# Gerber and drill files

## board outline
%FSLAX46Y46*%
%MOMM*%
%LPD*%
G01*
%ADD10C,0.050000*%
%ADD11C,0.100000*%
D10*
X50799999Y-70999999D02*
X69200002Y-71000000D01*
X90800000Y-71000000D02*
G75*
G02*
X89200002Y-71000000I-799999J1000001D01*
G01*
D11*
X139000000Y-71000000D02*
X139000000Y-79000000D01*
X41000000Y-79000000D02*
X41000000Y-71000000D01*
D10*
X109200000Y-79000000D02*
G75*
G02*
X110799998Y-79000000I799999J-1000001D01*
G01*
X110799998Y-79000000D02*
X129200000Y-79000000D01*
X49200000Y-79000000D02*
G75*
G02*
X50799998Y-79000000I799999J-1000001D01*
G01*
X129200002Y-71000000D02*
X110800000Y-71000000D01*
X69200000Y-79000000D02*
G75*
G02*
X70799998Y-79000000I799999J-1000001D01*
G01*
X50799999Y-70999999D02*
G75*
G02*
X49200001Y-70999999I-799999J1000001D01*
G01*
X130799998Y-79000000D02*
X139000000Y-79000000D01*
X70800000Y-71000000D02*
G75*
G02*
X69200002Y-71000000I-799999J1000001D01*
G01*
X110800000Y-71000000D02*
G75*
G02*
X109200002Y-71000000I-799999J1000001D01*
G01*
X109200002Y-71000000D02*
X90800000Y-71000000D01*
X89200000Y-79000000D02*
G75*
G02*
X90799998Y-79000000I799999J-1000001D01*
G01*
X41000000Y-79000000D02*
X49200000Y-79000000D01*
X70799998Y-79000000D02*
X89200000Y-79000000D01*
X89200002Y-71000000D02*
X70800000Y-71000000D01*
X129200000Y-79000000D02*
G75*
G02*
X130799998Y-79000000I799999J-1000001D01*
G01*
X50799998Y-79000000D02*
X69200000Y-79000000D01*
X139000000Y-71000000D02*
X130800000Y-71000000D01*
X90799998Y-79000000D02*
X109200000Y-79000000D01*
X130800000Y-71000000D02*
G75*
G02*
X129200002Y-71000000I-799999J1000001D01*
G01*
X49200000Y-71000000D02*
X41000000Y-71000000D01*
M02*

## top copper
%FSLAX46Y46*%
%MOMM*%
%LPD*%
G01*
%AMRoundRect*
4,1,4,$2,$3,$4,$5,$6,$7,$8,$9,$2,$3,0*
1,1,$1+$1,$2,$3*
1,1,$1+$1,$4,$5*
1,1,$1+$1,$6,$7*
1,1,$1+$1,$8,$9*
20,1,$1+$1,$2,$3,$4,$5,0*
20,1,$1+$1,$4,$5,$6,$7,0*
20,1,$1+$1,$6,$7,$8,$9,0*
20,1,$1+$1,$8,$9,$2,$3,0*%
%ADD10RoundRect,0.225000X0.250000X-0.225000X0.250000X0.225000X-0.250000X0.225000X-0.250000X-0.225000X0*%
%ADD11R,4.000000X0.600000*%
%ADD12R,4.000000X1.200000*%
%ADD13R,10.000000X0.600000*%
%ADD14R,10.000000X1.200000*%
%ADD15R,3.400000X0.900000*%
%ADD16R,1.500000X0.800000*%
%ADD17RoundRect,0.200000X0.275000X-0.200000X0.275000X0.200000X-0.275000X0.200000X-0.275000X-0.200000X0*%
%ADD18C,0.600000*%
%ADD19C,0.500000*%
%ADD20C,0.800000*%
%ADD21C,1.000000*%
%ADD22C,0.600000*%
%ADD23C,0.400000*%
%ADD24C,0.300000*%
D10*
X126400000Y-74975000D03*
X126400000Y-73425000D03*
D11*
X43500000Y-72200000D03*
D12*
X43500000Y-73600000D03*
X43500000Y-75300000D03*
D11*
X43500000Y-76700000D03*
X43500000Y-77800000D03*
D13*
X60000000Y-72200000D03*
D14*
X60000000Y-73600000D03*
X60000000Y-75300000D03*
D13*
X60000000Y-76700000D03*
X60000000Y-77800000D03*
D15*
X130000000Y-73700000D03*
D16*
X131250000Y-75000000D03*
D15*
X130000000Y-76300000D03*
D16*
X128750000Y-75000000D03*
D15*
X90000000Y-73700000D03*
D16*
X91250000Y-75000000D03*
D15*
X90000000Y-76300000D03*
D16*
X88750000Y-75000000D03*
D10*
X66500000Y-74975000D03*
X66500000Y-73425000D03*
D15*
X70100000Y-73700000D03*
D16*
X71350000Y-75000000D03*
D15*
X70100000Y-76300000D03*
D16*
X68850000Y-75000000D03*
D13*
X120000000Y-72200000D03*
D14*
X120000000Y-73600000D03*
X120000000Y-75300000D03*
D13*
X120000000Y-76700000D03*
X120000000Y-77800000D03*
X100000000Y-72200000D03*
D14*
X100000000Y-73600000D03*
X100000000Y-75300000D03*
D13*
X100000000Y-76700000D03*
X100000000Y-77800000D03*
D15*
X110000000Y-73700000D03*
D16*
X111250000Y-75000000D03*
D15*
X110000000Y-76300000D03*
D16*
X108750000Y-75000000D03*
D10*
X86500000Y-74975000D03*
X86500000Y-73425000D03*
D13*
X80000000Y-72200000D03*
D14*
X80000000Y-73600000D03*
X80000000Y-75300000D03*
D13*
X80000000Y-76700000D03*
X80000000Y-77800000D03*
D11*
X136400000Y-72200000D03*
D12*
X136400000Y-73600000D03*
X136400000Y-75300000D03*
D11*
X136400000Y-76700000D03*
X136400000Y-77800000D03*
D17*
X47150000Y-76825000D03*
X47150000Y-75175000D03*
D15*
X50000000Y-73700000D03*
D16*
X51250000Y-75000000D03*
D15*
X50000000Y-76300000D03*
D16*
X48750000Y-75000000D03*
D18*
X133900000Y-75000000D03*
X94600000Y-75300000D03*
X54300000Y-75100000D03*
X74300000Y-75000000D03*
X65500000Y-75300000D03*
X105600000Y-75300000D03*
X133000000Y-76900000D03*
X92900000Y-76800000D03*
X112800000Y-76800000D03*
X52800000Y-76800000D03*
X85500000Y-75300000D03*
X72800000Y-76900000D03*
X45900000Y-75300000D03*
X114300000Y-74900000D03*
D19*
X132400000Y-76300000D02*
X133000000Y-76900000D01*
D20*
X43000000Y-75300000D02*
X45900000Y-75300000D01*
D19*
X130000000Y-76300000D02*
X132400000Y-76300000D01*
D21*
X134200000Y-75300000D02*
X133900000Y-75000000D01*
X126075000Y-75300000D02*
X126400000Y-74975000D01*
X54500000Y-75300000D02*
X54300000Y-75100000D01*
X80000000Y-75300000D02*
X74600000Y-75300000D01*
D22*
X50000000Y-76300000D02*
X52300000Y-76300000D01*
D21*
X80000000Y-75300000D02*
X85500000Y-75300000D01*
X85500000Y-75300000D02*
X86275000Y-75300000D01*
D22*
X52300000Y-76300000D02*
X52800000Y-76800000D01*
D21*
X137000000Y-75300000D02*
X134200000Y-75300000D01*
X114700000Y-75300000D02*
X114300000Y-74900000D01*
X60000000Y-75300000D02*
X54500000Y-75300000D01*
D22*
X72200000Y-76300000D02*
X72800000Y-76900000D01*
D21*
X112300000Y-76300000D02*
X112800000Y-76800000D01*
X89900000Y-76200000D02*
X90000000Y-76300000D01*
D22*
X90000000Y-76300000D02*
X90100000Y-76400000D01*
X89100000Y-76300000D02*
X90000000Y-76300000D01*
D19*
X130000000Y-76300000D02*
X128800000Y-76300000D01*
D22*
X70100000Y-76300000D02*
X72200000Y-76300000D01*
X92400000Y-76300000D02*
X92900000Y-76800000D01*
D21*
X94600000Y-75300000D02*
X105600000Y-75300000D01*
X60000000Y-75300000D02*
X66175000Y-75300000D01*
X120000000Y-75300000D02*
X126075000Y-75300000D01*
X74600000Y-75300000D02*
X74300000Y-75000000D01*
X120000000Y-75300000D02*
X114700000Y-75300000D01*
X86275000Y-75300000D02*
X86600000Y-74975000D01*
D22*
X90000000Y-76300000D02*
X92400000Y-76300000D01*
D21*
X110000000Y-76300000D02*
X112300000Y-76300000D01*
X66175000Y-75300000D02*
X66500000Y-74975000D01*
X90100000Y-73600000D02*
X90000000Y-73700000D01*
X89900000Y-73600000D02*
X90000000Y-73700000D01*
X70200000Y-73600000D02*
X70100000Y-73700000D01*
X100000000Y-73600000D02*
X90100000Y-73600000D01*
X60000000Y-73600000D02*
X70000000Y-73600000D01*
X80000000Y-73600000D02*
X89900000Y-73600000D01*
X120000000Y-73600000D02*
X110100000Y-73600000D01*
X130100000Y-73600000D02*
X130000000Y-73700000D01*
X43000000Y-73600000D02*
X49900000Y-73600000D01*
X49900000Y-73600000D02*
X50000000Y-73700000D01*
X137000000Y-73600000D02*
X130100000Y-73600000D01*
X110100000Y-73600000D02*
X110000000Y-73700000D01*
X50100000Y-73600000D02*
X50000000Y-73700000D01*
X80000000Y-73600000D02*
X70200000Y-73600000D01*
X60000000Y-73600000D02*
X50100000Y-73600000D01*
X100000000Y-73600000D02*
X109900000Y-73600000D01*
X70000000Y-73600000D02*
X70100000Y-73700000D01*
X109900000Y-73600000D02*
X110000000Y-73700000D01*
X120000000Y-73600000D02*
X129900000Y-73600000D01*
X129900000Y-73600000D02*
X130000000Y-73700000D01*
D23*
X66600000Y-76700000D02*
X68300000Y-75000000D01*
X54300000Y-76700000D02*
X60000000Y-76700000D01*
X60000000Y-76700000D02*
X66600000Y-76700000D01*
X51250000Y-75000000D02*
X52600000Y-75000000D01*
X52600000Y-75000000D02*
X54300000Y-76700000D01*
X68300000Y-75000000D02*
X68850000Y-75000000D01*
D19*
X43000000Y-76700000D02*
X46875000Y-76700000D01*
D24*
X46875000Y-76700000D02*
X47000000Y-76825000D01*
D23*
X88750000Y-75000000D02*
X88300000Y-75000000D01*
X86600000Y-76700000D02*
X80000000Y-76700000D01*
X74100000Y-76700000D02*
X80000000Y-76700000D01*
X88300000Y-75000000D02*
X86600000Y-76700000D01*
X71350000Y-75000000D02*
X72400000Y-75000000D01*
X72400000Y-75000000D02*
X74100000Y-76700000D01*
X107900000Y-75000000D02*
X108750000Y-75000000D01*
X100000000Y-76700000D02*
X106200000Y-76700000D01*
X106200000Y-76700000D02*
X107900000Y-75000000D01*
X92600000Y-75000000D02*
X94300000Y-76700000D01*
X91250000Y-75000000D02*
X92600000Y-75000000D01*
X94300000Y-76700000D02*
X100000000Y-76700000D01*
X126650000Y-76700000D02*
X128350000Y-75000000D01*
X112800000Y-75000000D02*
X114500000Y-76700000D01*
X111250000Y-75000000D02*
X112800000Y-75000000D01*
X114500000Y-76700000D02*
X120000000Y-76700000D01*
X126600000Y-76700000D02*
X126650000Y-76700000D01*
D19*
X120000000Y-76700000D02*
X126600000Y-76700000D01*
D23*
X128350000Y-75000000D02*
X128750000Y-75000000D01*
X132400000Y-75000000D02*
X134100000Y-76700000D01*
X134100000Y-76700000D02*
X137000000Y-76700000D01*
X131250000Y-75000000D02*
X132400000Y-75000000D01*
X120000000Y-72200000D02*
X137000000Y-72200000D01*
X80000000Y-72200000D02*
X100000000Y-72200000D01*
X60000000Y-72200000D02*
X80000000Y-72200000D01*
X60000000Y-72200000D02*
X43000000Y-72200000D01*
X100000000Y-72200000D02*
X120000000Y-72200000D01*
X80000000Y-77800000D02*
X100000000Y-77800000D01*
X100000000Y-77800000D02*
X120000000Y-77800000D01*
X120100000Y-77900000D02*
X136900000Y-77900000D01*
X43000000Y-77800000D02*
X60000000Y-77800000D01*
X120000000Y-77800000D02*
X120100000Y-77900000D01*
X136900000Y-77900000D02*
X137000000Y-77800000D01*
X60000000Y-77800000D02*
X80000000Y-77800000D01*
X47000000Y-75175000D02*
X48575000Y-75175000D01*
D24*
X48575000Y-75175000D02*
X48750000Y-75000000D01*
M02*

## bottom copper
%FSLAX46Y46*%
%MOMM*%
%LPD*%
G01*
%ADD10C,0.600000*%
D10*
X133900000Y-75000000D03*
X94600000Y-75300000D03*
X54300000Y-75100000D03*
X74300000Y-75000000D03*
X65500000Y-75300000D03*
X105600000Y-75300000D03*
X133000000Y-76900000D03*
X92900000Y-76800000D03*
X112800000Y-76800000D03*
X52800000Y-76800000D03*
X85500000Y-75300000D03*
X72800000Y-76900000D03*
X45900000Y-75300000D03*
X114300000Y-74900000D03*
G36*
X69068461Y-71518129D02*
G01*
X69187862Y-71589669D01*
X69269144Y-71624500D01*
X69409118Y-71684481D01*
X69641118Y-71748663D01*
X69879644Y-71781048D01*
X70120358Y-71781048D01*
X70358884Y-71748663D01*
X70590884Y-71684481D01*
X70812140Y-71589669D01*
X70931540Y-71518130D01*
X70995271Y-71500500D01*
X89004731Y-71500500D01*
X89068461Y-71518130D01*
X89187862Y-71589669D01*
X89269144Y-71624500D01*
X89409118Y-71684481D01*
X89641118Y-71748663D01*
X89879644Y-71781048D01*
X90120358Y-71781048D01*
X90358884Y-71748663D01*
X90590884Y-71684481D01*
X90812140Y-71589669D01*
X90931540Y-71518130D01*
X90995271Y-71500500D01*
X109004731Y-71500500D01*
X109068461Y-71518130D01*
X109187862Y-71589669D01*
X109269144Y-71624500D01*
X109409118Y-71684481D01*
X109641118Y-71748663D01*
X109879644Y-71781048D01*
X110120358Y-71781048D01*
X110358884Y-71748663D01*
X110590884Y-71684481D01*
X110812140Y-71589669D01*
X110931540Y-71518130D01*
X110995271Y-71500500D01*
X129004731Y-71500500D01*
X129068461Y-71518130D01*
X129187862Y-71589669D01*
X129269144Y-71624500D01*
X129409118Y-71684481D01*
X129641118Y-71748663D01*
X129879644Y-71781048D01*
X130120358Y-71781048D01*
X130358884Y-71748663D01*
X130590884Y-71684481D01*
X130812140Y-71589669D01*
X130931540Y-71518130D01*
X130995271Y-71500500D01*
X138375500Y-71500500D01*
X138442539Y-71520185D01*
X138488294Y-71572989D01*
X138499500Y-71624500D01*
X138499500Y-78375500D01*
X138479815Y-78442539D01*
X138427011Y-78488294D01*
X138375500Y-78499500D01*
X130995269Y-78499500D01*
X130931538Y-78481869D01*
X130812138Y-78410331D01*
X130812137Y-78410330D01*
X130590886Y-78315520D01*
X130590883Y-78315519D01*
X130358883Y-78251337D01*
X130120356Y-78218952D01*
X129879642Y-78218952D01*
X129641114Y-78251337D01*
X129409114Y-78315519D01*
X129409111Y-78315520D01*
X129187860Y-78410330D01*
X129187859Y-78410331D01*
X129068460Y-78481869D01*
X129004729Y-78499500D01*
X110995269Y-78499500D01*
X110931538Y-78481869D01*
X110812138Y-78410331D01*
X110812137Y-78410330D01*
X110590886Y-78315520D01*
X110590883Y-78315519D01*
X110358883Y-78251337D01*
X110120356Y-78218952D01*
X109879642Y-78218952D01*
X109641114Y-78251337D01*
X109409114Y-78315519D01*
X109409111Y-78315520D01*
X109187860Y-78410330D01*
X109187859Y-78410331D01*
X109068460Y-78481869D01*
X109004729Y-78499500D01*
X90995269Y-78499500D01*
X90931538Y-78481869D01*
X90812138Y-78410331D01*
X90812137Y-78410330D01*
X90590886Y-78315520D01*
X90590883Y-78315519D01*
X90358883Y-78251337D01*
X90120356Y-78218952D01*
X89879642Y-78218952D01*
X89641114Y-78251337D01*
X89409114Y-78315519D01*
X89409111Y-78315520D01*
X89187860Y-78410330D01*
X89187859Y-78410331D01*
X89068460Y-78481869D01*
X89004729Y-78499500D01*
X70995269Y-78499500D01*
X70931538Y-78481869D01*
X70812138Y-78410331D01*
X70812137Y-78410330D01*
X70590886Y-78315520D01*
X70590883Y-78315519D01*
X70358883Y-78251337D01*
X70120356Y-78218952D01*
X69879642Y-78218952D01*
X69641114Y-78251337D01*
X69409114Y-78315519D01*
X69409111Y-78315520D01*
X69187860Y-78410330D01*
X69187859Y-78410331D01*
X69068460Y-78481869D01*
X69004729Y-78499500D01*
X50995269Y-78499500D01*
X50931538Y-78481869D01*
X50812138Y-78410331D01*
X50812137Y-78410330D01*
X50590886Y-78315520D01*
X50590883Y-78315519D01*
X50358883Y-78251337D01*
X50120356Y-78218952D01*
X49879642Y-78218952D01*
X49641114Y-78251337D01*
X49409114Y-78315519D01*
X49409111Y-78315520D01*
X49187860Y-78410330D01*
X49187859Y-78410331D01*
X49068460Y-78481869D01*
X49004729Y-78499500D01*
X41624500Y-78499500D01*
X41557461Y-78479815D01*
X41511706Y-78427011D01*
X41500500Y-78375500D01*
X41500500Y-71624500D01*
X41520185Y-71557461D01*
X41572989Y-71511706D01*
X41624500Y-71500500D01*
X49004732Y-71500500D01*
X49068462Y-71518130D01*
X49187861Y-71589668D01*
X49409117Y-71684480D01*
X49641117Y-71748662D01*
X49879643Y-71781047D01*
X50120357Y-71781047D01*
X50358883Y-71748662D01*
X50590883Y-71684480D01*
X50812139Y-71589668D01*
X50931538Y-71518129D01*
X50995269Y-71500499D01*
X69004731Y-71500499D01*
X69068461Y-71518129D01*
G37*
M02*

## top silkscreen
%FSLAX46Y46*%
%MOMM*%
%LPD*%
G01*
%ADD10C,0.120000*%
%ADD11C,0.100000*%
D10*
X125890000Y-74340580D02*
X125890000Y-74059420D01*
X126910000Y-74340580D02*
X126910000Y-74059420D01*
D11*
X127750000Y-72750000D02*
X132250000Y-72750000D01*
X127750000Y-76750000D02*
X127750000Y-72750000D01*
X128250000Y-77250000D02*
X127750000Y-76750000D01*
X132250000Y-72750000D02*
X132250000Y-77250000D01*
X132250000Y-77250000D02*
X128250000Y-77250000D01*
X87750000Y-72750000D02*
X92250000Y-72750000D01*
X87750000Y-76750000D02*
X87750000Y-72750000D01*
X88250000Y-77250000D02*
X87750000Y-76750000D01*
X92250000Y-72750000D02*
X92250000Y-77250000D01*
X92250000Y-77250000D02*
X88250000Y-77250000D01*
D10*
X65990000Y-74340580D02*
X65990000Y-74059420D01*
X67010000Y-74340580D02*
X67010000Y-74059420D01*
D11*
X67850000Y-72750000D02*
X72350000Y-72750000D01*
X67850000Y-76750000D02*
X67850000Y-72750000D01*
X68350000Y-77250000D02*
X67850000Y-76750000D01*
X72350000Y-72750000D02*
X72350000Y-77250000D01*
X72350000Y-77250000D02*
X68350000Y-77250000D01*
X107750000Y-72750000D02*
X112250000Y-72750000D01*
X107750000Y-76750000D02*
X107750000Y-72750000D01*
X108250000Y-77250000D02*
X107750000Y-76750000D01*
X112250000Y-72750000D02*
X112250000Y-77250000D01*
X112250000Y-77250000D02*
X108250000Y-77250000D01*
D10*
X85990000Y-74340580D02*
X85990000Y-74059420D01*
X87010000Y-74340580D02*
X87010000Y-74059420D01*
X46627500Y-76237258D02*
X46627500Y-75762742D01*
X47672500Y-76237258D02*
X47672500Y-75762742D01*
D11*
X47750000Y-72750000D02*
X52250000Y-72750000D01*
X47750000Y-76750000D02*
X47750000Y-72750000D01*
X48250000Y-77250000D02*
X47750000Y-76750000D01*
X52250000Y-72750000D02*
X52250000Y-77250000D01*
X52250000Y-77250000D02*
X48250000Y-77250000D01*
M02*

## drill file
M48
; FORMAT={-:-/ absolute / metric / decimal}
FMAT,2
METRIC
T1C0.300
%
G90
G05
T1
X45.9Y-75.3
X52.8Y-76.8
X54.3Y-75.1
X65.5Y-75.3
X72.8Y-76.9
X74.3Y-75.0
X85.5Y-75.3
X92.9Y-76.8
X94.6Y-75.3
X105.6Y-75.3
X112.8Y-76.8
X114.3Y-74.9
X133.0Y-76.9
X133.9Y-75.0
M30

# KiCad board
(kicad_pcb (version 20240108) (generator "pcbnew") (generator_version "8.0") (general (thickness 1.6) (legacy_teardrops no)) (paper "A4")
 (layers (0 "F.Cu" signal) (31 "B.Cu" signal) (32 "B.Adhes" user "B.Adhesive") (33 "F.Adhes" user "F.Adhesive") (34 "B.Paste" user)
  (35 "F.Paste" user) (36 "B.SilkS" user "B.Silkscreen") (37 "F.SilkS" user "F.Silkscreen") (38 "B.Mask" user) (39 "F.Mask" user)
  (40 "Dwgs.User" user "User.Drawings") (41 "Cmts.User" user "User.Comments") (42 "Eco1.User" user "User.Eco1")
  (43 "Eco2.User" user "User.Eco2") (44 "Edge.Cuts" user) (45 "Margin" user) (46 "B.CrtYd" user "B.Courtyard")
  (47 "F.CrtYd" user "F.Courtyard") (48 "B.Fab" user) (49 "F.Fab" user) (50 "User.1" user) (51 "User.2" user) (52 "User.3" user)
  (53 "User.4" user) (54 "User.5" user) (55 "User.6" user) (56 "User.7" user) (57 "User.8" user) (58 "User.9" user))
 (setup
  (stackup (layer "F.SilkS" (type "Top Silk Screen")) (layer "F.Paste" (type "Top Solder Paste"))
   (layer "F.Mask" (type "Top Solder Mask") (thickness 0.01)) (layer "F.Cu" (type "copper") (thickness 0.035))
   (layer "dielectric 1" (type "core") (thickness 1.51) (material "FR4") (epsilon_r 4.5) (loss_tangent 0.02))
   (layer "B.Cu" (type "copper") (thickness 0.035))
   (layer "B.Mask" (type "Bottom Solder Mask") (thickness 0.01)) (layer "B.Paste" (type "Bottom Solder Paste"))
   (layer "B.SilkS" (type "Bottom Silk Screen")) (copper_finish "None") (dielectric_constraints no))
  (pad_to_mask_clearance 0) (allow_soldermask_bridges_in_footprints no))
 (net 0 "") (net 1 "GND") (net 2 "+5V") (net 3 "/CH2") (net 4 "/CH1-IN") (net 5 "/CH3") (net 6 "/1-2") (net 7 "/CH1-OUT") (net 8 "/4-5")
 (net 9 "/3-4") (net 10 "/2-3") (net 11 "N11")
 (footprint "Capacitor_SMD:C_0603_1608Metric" (layer "F.Cu") (at 126.4 74.2 90)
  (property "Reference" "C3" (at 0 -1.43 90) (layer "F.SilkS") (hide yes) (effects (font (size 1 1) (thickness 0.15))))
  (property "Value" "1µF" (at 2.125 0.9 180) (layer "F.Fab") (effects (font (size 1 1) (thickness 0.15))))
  (fp_line (start -0.14058 -0.51) (end 0.14058 -0.51) (stroke (width 0.12) (type solid)) (layer "F.SilkS"))
  (fp_line (start -0.14058 0.51) (end 0.14058 0.51) (stroke (width 0.12) (type solid)) (layer "F.SilkS"))
  (pad "1" smd roundrect (at -0.775 0 90) (size 0.9 0.95) (layers "F.Cu" "F.Paste" "F.Mask") (roundrect_rratio 0.25) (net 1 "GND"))
  (pad "2" smd roundrect (at 0.775 0 90) (size 0.9 0.95) (layers "F.Cu" "F.Paste" "F.Mask") (roundrect_rratio 0.25) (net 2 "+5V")))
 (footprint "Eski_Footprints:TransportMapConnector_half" (layer "F.Cu") (at 43.5 75)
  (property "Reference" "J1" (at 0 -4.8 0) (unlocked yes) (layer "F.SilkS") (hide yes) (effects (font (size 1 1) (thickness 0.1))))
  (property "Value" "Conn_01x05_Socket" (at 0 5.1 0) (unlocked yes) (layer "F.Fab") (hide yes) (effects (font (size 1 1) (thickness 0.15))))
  (pad "1" smd rect (at 0 -2.8) (size 4 0.6) (layers "F.Cu" "F.Paste" "F.Mask") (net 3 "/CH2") (thermal_bridge_angle 45))
  (pad "2" smd rect (at 0 -1.4) (size 4 1.2) (layers "F.Cu" "F.Paste" "F.Mask") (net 2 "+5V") (thermal_bridge_angle 45))
  (pad "3" smd rect (at 0 0.3) (size 4 1.2) (layers "F.Cu" "F.Paste" "F.Mask") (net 1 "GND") (thermal_bridge_angle 45))
  (pad "4" smd rect (at 0 1.7) (size 4 0.6) (layers "F.Cu" "F.Paste" "F.Mask") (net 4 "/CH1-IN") (thermal_bridge_angle 45))
  (pad "5" smd rect (at 0 2.8) (size 4 0.6) (layers "F.Cu" "F.Paste" "F.Mask") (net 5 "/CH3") (thermal_bridge_angle 45)))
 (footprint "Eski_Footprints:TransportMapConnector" (layer "F.Cu") (at 60 75)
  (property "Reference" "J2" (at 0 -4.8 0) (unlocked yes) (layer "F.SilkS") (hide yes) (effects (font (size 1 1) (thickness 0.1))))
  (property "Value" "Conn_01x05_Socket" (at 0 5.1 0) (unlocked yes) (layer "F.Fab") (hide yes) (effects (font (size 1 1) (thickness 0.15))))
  (pad "1" smd rect (at 0 -2.8) (size 10 0.6) (layers "F.Cu" "F.Paste" "F.Mask") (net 3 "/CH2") (thermal_bridge_angle 45))
  (pad "2" smd rect (at 0 -1.4) (size 10 1.2) (layers "F.Cu" "F.Paste" "F.Mask") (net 2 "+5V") (thermal_bridge_angle 45))
  (pad "3" smd rect (at 0 0.3) (size 10 1.2) (layers "F.Cu" "F.Paste" "F.Mask") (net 1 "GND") (thermal_bridge_angle 45))
  (pad "4" smd rect (at 0 1.7) (size 10 0.6) (layers "F.Cu" "F.Paste" "F.Mask") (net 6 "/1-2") (thermal_bridge_angle 45))
  (pad "5" smd rect (at 0 2.8) (size 10 0.6) (layers "F.Cu" "F.Paste" "F.Mask") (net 5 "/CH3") (thermal_bridge_angle 45)))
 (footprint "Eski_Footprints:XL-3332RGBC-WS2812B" (layer "F.Cu") (at 130 75)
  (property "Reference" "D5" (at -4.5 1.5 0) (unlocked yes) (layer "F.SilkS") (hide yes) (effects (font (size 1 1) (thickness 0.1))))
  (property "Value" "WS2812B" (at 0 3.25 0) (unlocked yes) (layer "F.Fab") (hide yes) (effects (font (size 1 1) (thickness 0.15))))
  (fp_line (start -2.25 -2.25) (end 2.25 -2.25) (stroke (width 0.1) (type default)) (layer "F.SilkS"))
  (fp_line (start -2.25 1.75) (end -2.25 -2.25) (stroke (width 0.1) (type default)) (layer "F.SilkS"))
  (fp_line (start -1.75 2.25) (end -2.25 1.75) (stroke (width 0.1) (type default)) (layer "F.SilkS"))
  (fp_line (start 2.25 -2.25) (end 2.25 2.25) (stroke (width 0.1) (type default)) (layer "F.SilkS"))
  (fp_line (start 2.25 2.25) (end -1.75 2.25) (stroke (width 0.1) (type default)) (layer "F.SilkS"))
  (pad "1" smd rect (at 0 -1.3) (size 3.4 0.9) (layers "F.Cu" "F.Paste" "F.Mask") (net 2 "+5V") (thermal_bridge_angle 45))
  (pad "2" smd rect (at 1.25 0) (size 1.5 0.8) (layers "F.Cu" "F.Paste" "F.Mask") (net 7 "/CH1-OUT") (thermal_bridge_angle 45))
  (pad "3" smd rect (at 0 1.3) (size 3.4 0.9) (layers "F.Cu" "F.Paste" "F.Mask") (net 1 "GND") (thermal_bridge_angle 45))
  (pad "4" smd rect (at -1.25 0) (size 1.5 0.8) (layers "F.Cu" "F.Paste" "F.Mask") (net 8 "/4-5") (thermal_bridge_angle 45)))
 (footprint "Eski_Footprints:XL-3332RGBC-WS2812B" (layer "F.Cu") (at 90 75)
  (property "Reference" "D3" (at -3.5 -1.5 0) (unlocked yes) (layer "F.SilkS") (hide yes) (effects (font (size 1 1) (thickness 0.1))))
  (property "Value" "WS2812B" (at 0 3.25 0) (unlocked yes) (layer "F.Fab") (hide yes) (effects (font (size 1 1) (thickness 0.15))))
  (fp_line (start -2.25 -2.25) (end 2.25 -2.25) (stroke (width 0.1) (type default)) (layer "F.SilkS"))
  (fp_line (start -2.25 1.75) (end -2.25 -2.25) (stroke (width 0.1) (type default)) (layer "F.SilkS"))
  (fp_line (start -1.75 2.25) (end -2.25 1.75) (stroke (width 0.1) (type default)) (layer "F.SilkS"))
  (fp_line (start 2.25 -2.25) (end 2.25 2.25) (stroke (width 0.1) (type default)) (layer "F.SilkS"))
  (fp_line (start 2.25 2.25) (end -1.75 2.25) (stroke (width 0.1) (type default)) (layer "F.SilkS"))
  (pad "1" smd rect (at 0 -1.3) (size 3.4 0.9) (layers "F.Cu" "F.Paste" "F.Mask") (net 2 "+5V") (thermal_bridge_angle 45))
  (pad "2" smd rect (at 1.25 0) (size 1.5 0.8) (layers "F.Cu" "F.Paste" "F.Mask") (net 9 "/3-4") (thermal_bridge_angle 45))
  (pad "3" smd rect (at 0 1.3) (size 3.4 0.9) (layers "F.Cu" "F.Paste" "F.Mask") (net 1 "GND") (thermal_bridge_angle 45))
  (pad "4" smd rect (at -1.25 0) (size 1.5 0.8) (layers "F.Cu" "F.Paste" "F.Mask") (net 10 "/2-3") (thermal_bridge_angle 45)))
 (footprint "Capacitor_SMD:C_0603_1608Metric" (layer "F.Cu") (at 66.5 74.2 90)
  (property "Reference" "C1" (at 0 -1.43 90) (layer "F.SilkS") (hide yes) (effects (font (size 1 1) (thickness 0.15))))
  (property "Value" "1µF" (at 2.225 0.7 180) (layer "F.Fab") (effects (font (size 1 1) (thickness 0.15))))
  (fp_line (start -0.14058 -0.51) (end 0.14058 -0.51) (stroke (width 0.12) (type solid)) (layer "F.SilkS"))
  (fp_line (start -0.14058 0.51) (end 0.14058 0.51) (stroke (width 0.12) (type solid)) (layer "F.SilkS"))
  (pad "1" smd roundrect (at -0.775 0 90) (size 0.9 0.95) (layers "F.Cu" "F.Paste" "F.Mask") (roundrect_rratio 0.25) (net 1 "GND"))
  (pad "2" smd roundrect (at 0.775 0 90) (size 0.9 0.95) (layers "F.Cu" "F.Paste" "F.Mask") (roundrect_rratio 0.25) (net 2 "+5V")))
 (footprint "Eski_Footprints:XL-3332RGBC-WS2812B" (layer "F.Cu") (at 70.1 75)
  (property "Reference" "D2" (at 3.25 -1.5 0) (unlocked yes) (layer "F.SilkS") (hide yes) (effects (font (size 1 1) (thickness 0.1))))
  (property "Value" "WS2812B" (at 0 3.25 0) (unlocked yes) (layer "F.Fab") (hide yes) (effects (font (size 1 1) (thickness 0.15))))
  (fp_line (start -2.25 -2.25) (end 2.25 -2.25) (stroke (width 0.1) (type default)) (layer "F.SilkS"))
  (fp_line (start -2.25 1.75) (end -2.25 -2.25) (stroke (width 0.1) (type default)) (layer "F.SilkS"))
  (fp_line (start -1.75 2.25) (end -2.25 1.75) (stroke (width 0.1) (type default)) (layer "F.SilkS"))
  (fp_line (start 2.25 -2.25) (end 2.25 2.25) (stroke (width 0.1) (type default)) (layer "F.SilkS"))
  (fp_line (start 2.25 2.25) (end -1.75 2.25) (stroke (width 0.1) (type default)) (layer "F.SilkS"))
  (pad "1" smd rect (at 0 -1.3) (size 3.4 0.9) (layers "F.Cu" "F.Paste" "F.Mask") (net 2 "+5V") (thermal_bridge_angle 45))
  (pad "2" smd rect (at 1.25 0) (size 1.5 0.8) (layers "F.Cu" "F.Paste" "F.Mask") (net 10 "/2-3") (thermal_bridge_angle 45))
  (pad "3" smd rect (at 0 1.3) (size 3.4 0.9) (layers "F.Cu" "F.Paste" "F.Mask") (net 1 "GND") (thermal_bridge_angle 45))
  (pad "4" smd rect (at -1.25 0) (size 1.5 0.8) (layers "F.Cu" "F.Paste" "F.Mask") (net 6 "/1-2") (thermal_bridge_angle 45)))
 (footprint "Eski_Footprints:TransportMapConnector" (layer "F.Cu") (at 120 75)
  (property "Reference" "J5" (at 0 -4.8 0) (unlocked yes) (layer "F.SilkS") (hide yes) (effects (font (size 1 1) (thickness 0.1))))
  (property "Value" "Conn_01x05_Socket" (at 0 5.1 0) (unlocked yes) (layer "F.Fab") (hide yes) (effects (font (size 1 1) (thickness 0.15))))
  (pad "1" smd rect (at 0 -2.8) (size 10 0.6) (layers "F.Cu" "F.Paste" "F.Mask") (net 3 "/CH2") (thermal_bridge_angle 45))
  (pad "2" smd rect (at 0 -1.4) (size 10 1.2) (layers "F.Cu" "F.Paste" "F.Mask") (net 2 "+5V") (thermal_bridge_angle 45))
  (pad "3" smd rect (at 0 0.3) (size 10 1.2) (layers "F.Cu" "F.Paste" "F.Mask") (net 1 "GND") (thermal_bridge_angle 45))
  (pad "4" smd rect (at 0 1.7) (size 10 0.6) (layers "F.Cu" "F.Paste" "F.Mask") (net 8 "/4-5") (thermal_bridge_angle 45))
  (pad "5" smd rect (at 0 2.8) (size 10 0.6) (layers "F.Cu" "F.Paste" "F.Mask") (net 5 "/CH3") (thermal_bridge_angle 45)))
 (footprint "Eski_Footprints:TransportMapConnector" (layer "F.Cu") (at 100 75)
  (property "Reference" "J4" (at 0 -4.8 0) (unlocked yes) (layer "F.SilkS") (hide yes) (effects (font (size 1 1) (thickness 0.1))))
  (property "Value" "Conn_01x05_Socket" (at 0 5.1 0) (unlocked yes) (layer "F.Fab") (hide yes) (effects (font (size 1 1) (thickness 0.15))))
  (pad "1" smd rect (at 0 -2.8) (size 10 0.6) (layers "F.Cu" "F.Paste" "F.Mask") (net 3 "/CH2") (thermal_bridge_angle 45))
  (pad "2" smd rect (at 0 -1.4) (size 10 1.2) (layers "F.Cu" "F.Paste" "F.Mask") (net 2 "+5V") (thermal_bridge_angle 45))
  (pad "3" smd rect (at 0 0.3) (size 10 1.2) (layers "F.Cu" "F.Paste" "F.Mask") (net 1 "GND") (thermal_bridge_angle 45))
  (pad "4" smd rect (at 0 1.7) (size 10 0.6) (layers "F.Cu" "F.Paste" "F.Mask") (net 9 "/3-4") (thermal_bridge_angle 45))
  (pad "5" smd rect (at 0 2.8) (size 10 0.6) (layers "F.Cu" "F.Paste" "F.Mask") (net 5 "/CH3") (thermal_bridge_angle 45)))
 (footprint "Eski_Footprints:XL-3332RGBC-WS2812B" (layer "F.Cu") (at 110 75)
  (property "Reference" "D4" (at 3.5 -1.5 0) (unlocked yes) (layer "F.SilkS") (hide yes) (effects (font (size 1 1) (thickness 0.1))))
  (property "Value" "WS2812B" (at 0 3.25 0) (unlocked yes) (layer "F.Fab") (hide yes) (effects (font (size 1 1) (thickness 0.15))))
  (fp_line (start -2.25 -2.25) (end 2.25 -2.25) (stroke (width 0.1) (type default)) (layer "F.SilkS"))
  (fp_line (start -2.25 1.75) (end -2.25 -2.25) (stroke (width 0.1) (type default)) (layer "F.SilkS"))
  (fp_line (start -1.75 2.25) (end -2.25 1.75) (stroke (width 0.1) (type default)) (layer "F.SilkS"))
  (fp_line (start 2.25 -2.25) (end 2.25 2.25) (stroke (width 0.1) (type default)) (layer "F.SilkS"))
  (fp_line (start 2.25 2.25) (end -1.75 2.25) (stroke (width 0.1) (type default)) (layer "F.SilkS"))
  (pad "1" smd rect (at 0 -1.3) (size 3.4 0.9) (layers "F.Cu" "F.Paste" "F.Mask") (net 2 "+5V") (thermal_bridge_angle 45))
  (pad "2" smd rect (at 1.25 0) (size 1.5 0.8) (layers "F.Cu" "F.Paste" "F.Mask") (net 8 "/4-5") (thermal_bridge_angle 45))
  (pad "3" smd rect (at 0 1.3) (size 3.4 0.9) (layers "F.Cu" "F.Paste" "F.Mask") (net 1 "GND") (thermal_bridge_angle 45))
  (pad "4" smd rect (at -1.25 0) (size 1.5 0.8) (layers "F.Cu" "F.Paste" "F.Mask") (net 9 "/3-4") (thermal_bridge_angle 45)))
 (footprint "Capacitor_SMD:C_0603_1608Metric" (layer "F.Cu") (at 86.5 74.2 90)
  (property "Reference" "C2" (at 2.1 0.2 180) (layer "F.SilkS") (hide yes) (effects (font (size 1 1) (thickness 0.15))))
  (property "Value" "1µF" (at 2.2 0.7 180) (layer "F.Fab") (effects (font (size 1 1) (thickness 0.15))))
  (fp_line (start -0.14058 -0.51) (end 0.14058 -0.51) (stroke (width 0.12) (type solid)) (layer "F.SilkS"))
  (fp_line (start -0.14058 0.51) (end 0.14058 0.51) (stroke (width 0.12) (type solid)) (layer "F.SilkS"))
  (pad "1" smd roundrect (at -0.775 0 90) (size 0.9 0.95) (layers "F.Cu" "F.Paste" "F.Mask") (roundrect_rratio 0.25) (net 1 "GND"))
  (pad "2" smd roundrect (at 0.775 0 90) (size 0.9 0.95) (layers "F.Cu" "F.Paste" "F.Mask") (roundrect_rratio 0.25) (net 2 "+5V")))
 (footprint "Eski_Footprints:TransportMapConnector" (layer "F.Cu") (at 80 75)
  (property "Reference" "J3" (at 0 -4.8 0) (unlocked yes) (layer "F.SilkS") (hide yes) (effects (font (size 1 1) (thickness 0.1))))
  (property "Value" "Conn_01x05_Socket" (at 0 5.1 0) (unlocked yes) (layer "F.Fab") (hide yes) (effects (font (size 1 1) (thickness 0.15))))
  (pad "1" smd rect (at 0 -2.8) (size 10 0.6) (layers "F.Cu" "F.Paste" "F.Mask") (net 3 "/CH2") (thermal_bridge_angle 45))
  (pad "2" smd rect (at 0 -1.4) (size 10 1.2) (layers "F.Cu" "F.Paste" "F.Mask") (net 2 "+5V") (thermal_bridge_angle 45))
  (pad "3" smd rect (at 0 0.3) (size 10 1.2) (layers "F.Cu" "F.Paste" "F.Mask") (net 1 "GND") (thermal_bridge_angle 45))
  (pad "4" smd rect (at 0 1.7) (size 10 0.6) (layers "F.Cu" "F.Paste" "F.Mask") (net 10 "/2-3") (thermal_bridge_angle 45))
  (pad "5" smd rect (at 0 2.8) (size 10 0.6) (layers "F.Cu" "F.Paste" "F.Mask") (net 5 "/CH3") (thermal_bridge_angle 45)))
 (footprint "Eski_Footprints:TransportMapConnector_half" (layer "F.Cu") (at 136.4 75)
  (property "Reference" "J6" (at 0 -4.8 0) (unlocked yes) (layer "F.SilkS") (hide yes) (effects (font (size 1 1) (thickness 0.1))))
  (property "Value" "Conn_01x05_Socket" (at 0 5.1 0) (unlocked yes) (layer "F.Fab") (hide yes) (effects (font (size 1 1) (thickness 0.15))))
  (pad "1" smd rect (at 0 -2.8) (size 4 0.6) (layers "F.Cu" "F.Paste" "F.Mask") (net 3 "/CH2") (thermal_bridge_angle 45))
  (pad "2" smd rect (at 0 -1.4) (size 4 1.2) (layers "F.Cu" "F.Paste" "F.Mask") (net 2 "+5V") (thermal_bridge_angle 45))
  (pad "3" smd rect (at 0 0.3) (size 4 1.2) (layers "F.Cu" "F.Paste" "F.Mask") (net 1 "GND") (thermal_bridge_angle 45))
  (pad "4" smd rect (at 0 1.7) (size 4 0.6) (layers "F.Cu" "F.Paste" "F.Mask") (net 7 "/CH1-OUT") (thermal_bridge_angle 45))
  (pad "5" smd rect (at 0 2.8) (size 4 0.6) (layers "F.Cu" "F.Paste" "F.Mask") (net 5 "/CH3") (thermal_bridge_angle 45)))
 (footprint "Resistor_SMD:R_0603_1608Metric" (layer "F.Cu") (at 47.15 76 90)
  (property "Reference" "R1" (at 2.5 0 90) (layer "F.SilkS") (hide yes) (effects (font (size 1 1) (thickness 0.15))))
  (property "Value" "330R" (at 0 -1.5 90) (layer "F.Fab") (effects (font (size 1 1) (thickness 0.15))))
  (fp_line (start -0.237258 -0.5225) (end 0.237258 -0.5225) (stroke (width 0.12) (type solid)) (layer "F.SilkS"))
  (fp_line (start -0.237258 0.5225) (end 0.237258 0.5225) (stroke (width 0.12) (type solid)) (layer "F.SilkS"))
  (pad "1" smd roundrect (at -0.825 0 90) (size 0.8 0.95) (layers "F.Cu" "F.Paste" "F.Mask") (roundrect_rratio 0.25) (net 4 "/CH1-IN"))
  (pad "2" smd roundrect (at 0.825 0 90) (size 0.8 0.95) (layers "F.Cu" "F.Paste" "F.Mask") (roundrect_rratio 0.25) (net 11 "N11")))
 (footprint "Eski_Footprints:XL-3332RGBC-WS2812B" (layer "F.Cu") (at 50 75)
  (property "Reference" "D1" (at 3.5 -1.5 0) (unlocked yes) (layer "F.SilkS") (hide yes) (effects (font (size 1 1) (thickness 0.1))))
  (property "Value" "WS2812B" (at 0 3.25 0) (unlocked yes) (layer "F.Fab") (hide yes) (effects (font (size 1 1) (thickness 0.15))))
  (fp_line (start -2.25 -2.25) (end 2.25 -2.25) (stroke (width 0.1) (type default)) (layer "F.SilkS"))
  (fp_line (start -2.25 1.75) (end -2.25 -2.25) (stroke (width 0.1) (type default)) (layer "F.SilkS"))
  (fp_line (start -1.75 2.25) (end -2.25 1.75) (stroke (width 0.1) (type default)) (layer "F.SilkS"))
  (fp_line (start 2.25 -2.25) (end 2.25 2.25) (stroke (width 0.1) (type default)) (layer "F.SilkS"))
  (fp_line (start 2.25 2.25) (end -1.75 2.25) (stroke (width 0.1) (type default)) (layer "F.SilkS"))
  (pad "1" smd rect (at 0 -1.3) (size 3.4 0.9) (layers "F.Cu" "F.Paste" "F.Mask") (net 2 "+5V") (thermal_bridge_angle 45))
  (pad "2" smd rect (at 1.25 0) (size 1.5 0.8) (layers "F.Cu" "F.Paste" "F.Mask") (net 6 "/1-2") (thermal_bridge_angle 45))
  (pad "3" smd rect (at 0 1.3) (size 3.4 0.9) (layers "F.Cu" "F.Paste" "F.Mask") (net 1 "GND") (thermal_bridge_angle 45))
  (pad "4" smd rect (at -1.25 0) (size 1.5 0.8) (layers "F.Cu" "F.Paste" "F.Mask") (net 11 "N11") (thermal_bridge_angle 45)))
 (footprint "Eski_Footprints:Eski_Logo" (layer "B.Cu") (at 60.1 76.6 180)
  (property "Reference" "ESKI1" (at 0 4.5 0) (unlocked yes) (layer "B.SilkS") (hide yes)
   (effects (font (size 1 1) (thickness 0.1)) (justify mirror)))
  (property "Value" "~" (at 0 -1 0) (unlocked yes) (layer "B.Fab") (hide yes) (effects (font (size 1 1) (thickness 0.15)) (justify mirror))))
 (gr_line (start 50.799999 70.999999) (end 69.200002 71) (stroke (width 0.05) (type default)) (layer "Edge.Cuts"))
 (gr_arc (start 90.8 71) (mid 90.000001 71.280624) (end 89.200002 71) (stroke (width 0.05) (type default)) (layer "Edge.Cuts"))
 (gr_line (start 139 71) (end 139 79) (stroke (width 0.1) (type default)) (layer "Edge.Cuts"))
 (gr_line (start 41 79) (end 41 71) (stroke (width 0.1) (type default)) (layer "Edge.Cuts"))
 (gr_arc (start 109.2 79) (mid 109.999999 78.719376) (end 110.799998 79) (stroke (width 0.05) (type default)) (layer "Edge.Cuts"))
 (gr_line (start 110.799998 79) (end 129.2 79) (stroke (width 0.05) (type default)) (layer "Edge.Cuts"))
 (gr_arc (start 49.2 79) (mid 49.999999 78.719376) (end 50.799998 79) (stroke (width 0.05) (type default)) (layer "Edge.Cuts"))
 (gr_line (start 129.200002 71) (end 110.8 71) (stroke (width 0.05) (type default)) (layer "Edge.Cuts"))
 (gr_arc (start 69.2 79) (mid 69.999999 78.719376) (end 70.799998 79) (stroke (width 0.05) (type default)) (layer "Edge.Cuts"))
 (gr_arc (start 50.799999 70.999999) (mid 50 71.280623) (end 49.200001 70.999999) (stroke (width 0.05) (type default)) (layer "Edge.Cuts"))
 (gr_line (start 130.799998 79) (end 139 79) (stroke (width 0.05) (type default)) (layer "Edge.Cuts"))
 (gr_arc (start 70.8 71) (mid 70.000001 71.280624) (end 69.200002 71) (stroke (width 0.05) (type default)) (layer "Edge.Cuts"))
 (gr_arc (start 110.8 71) (mid 110.000001 71.280624) (end 109.200002 71) (stroke (width 0.05) (type default)) (layer "Edge.Cuts"))
 (gr_line (start 109.200002 71) (end 90.8 71) (stroke (width 0.05) (type default)) (layer "Edge.Cuts"))
 (gr_arc (start 89.2 79) (mid 89.999999 78.719376) (end 90.799998 79) (stroke (width 0.05) (type default)) (layer "Edge.Cuts"))
 (gr_line (start 41 79) (end 49.2 79) (stroke (width 0.05) (type default)) (layer "Edge.Cuts"))
 (gr_line (start 70.799998 79) (end 89.2 79) (stroke (width 0.05) (type default)) (layer "Edge.Cuts"))
 (gr_line (start 89.200002 71) (end 70.8 71) (stroke (width 0.05) (type default)) (layer "Edge.Cuts"))
 (gr_arc (start 129.2 79) (mid 129.999999 78.719376) (end 130.799998 79) (stroke (width 0.05) (type default)) (layer "Edge.Cuts"))
 (gr_line (start 50.799998 79) (end 69.2 79) (stroke (width 0.05) (type default)) (layer "Edge.Cuts"))
 (gr_line (start 139 71) (end 130.8 71) (stroke (width 0.05) (type default)) (layer "Edge.Cuts"))
 (gr_line (start 90.799998 79) (end 109.2 79) (stroke (width 0.05) (type default)) (layer "Edge.Cuts"))
 (gr_arc (start 130.8 71) (mid 130.000001 71.280624) (end 129.200002 71) (stroke (width 0.05) (type default)) (layer "Edge.Cuts"))
 (gr_line (start 49.2 71) (end 41 71) (stroke (width 0.05) (type default)) (layer "Edge.Cuts"))
 (segment (start 132.4 76.3) (end 133 76.9) (width 0.5) (layer "F.Cu") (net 1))
 (segment (start 43 75.3) (end 45.9 75.3) (width 0.8) (layer "F.Cu") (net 1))
 (segment (start 130 76.3) (end 132.4 76.3) (width 0.5) (layer "F.Cu") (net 1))
 (segment (start 134.2 75.3) (end 133.9 75) (width 1) (layer "F.Cu") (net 1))
 (segment (start 126.075 75.3) (end 126.4 74.975) (width 1) (layer "F.Cu") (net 1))
 (segment (start 54.5 75.3) (end 54.3 75.1) (width 1) (layer "F.Cu") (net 1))
 (segment (start 80 75.3) (end 74.6 75.3) (width 1) (layer "F.Cu") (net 1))
 (segment (start 50 76.3) (end 52.3 76.3) (width 0.6) (layer "F.Cu") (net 1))
 (segment (start 80 75.3) (end 85.5 75.3) (width 1) (layer "F.Cu") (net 1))
 (segment (start 85.5 75.3) (end 86.275 75.3) (width 1) (layer "F.Cu") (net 1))
 (segment (start 52.3 76.3) (end 52.8 76.8) (width 0.6) (layer "F.Cu") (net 1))
 (segment (start 137 75.3) (end 134.2 75.3) (width 1) (layer "F.Cu") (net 1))
 (segment (start 114.7 75.3) (end 114.3 74.9) (width 1) (layer "F.Cu") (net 1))
 (segment (start 60 75.3) (end 54.5 75.3) (width 1) (layer "F.Cu") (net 1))
 (segment (start 72.2 76.3) (end 72.8 76.9) (width 0.6) (layer "F.Cu") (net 1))
 (segment (start 112.3 76.3) (end 112.8 76.8) (width 1) (layer "F.Cu") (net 1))
 (segment (start 89.9 76.2) (end 90 76.3) (width 1) (layer "F.Cu") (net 1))
 (segment (start 90 76.3) (end 90.1 76.4) (width 0.6) (layer "F.Cu") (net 1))
 (segment (start 89.1 76.3) (end 90 76.3) (width 0.6) (layer "F.Cu") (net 1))
 (segment (start 130 76.3) (end 128.8 76.3) (width 0.5) (layer "F.Cu") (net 1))
 (segment (start 70.1 76.3) (end 72.2 76.3) (width 0.6) (layer "F.Cu") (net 1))
 (segment (start 92.4 76.3) (end 92.9 76.8) (width 0.6) (layer "F.Cu") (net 1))
 (segment (start 94.6 75.3) (end 105.6 75.3) (width 1) (layer "F.Cu") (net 1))
 (segment (start 60 75.3) (end 66.175 75.3) (width 1) (layer "F.Cu") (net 1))
 (segment (start 120 75.3) (end 126.075 75.3) (width 1) (layer "F.Cu") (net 1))
 (segment (start 74.6 75.3) (end 74.3 75) (width 1) (layer "F.Cu") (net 1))
 (segment (start 120 75.3) (end 114.7 75.3) (width 1) (layer "F.Cu") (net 1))
 (segment (start 86.275 75.3) (end 86.6 74.975) (width 1) (layer "F.Cu") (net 1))
 (segment (start 90 76.3) (end 92.4 76.3) (width 0.6) (layer "F.Cu") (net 1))
 (segment (start 110 76.3) (end 112.3 76.3) (width 1) (layer "F.Cu") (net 1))
 (segment (start 66.175 75.3) (end 66.5 74.975) (width 1) (layer "F.Cu") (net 1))
 (via (at 133.9 75) (size 0.6) (drill 0.3) (layers "F.Cu" "B.Cu") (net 1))
 (via (at 94.6 75.3) (size 0.6) (drill 0.3) (layers "F.Cu" "B.Cu") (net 1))
 (via (at 54.3 75.1) (size 0.6) (drill 0.3) (layers "F.Cu" "B.Cu") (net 1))
 (via (at 74.3 75) (size 0.6) (drill 0.3) (layers "F.Cu" "B.Cu") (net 1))
 (via (at 65.5 75.3) (size 0.6) (drill 0.3) (layers "F.Cu" "B.Cu") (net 1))
 (via (at 105.6 75.3) (size 0.6) (drill 0.3) (layers "F.Cu" "B.Cu") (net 1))
 (via (at 133 76.9) (size 0.6) (drill 0.3) (layers "F.Cu" "B.Cu") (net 1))
 (via (at 92.9 76.8) (size 0.6) (drill 0.3) (layers "F.Cu" "B.Cu") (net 1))
 (via (at 112.8 76.8) (size 0.6) (drill 0.3) (layers "F.Cu" "B.Cu") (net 1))
 (via (at 52.8 76.8) (size 0.6) (drill 0.3) (layers "F.Cu" "B.Cu") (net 1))
 (via (at 85.5 75.3) (size 0.6) (drill 0.3) (layers "F.Cu" "B.Cu") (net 1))
 (via (at 72.8 76.9) (size 0.6) (drill 0.3) (layers "F.Cu" "B.Cu") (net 1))
 (via (at 45.9 75.3) (size 0.6) (drill 0.3) (layers "F.Cu" "B.Cu") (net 1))
 (via (at 114.3 74.9) (size 0.6) (drill 0.3) (layers "F.Cu" "B.Cu") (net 1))
 (segment (start 90.1 73.6) (end 90 73.7) (width 1) (layer "F.Cu") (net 2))
 (segment (start 89.9 73.6) (end 90 73.7) (width 1) (layer "F.Cu") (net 2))
 (segment (start 70.2 73.6) (end 70.1 73.7) (width 1) (layer "F.Cu") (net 2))
 (segment (start 100 73.6) (end 90.1 73.6) (width 1) (layer "F.Cu") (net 2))
 (segment (start 60 73.6) (end 70 73.6) (width 1) (layer "F.Cu") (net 2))
 (segment (start 80 73.6) (end 89.9 73.6) (width 1) (layer "F.Cu") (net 2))
 (segment (start 120 73.6) (end 110.1 73.6) (width 1) (layer "F.Cu") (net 2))
 (segment (start 130.1 73.6) (end 130 73.7) (width 1) (layer "F.Cu") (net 2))
 (segment (start 43 73.6) (end 49.9 73.6) (width 1) (layer "F.Cu") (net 2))
 (segment (start 49.9 73.6) (end 50 73.7) (width 1) (layer "F.Cu") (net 2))
 (segment (start 137 73.6) (end 130.1 73.6) (width 1) (layer "F.Cu") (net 2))
 (segment (start 110.1 73.6) (end 110 73.7) (width 1) (layer "F.Cu") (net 2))
 (segment (start 50.1 73.6) (end 50 73.7) (width 1) (layer "F.Cu") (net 2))
 (segment (start 80 73.6) (end 70.2 73.6) (width 1) (layer "F.Cu") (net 2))
 (segment (start 60 73.6) (end 50.1 73.6) (width 1) (layer "F.Cu") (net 2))
 (segment (start 100 73.6) (end 109.9 73.6) (width 1) (layer "F.Cu") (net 2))
 (segment (start 70 73.6) (end 70.1 73.7) (width 1) (layer "F.Cu") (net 2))
 (segment (start 109.9 73.6) (end 110 73.7) (width 1) (layer "F.Cu") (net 2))
 (segment (start 120 73.6) (end 129.9 73.6) (width 1) (layer "F.Cu") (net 2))
 (segment (start 129.9 73.6) (end 130 73.7) (width 1) (layer "F.Cu") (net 2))
 (segment (start 66.6 76.7) (end 68.3 75) (width 0.4) (layer "F.Cu") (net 6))
 (segment (start 54.3 76.7) (end 60 76.7) (width 0.4) (layer "F.Cu") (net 6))
 (segment (start 60 76.7) (end 66.6 76.7) (width 0.4) (layer "F.Cu") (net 6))
 (segment (start 51.25 75) (end 52.6 75) (width 0.4) (layer "F.Cu") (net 6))
 (segment (start 52.6 75) (end 54.3 76.7) (width 0.4) (layer "F.Cu") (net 6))
 (segment (start 68.3 75) (end 68.85 75) (width 0.4) (layer "F.Cu") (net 6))
 (segment (start 43 76.7) (end 46.875 76.7) (width 0.5) (layer "F.Cu") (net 4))
 (segment (start 46.875 76.7) (end 47 76.825) (width 0.3) (layer "F.Cu") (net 4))
 (segment (start 88.75 75) (end 88.3 75) (width 0.4) (layer "F.Cu") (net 10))
 (segment (start 86.6 76.7) (end 80 76.7) (width 0.4) (layer "F.Cu") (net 10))
 (segment (start 74.1 76.7) (end 80 76.7) (width 0.4) (layer "F.Cu") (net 10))
 (segment (start 88.3 75) (end 86.6 76.7) (width 0.4) (layer "F.Cu") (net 10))
 (segment (start 71.35 75) (end 72.4 75) (width 0.4) (layer "F.Cu") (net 10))
 (segment (start 72.4 75) (end 74.1 76.7) (width 0.4) (layer "F.Cu") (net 10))
 (segment (start 107.9 75) (end 108.75 75) (width 0.4) (layer "F.Cu") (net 9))
 (segment (start 100 76.7) (end 106.2 76.7) (width 0.4) (layer "F.Cu") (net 9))
 (segment (start 106.2 76.7) (end 107.9 75) (width 0.4) (layer "F.Cu") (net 9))
 (segment (start 92.6 75) (end 94.3 76.7) (width 0.4) (layer "F.Cu") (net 9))
 (segment (start 91.25 75) (end 92.6 75) (width 0.4) (layer "F.Cu") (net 9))
 (segment (start 94.3 76.7) (end 100 76.7) (width 0.4) (layer "F.Cu") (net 9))
 (segment (start 126.65 76.7) (end 128.35 75) (width 0.4) (layer "F.Cu") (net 8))
 (segment (start 112.8 75) (end 114.5 76.7) (width 0.4) (layer "F.Cu") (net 8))
 (segment (start 111.25 75) (end 112.8 75) (width 0.4) (layer "F.Cu") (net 8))
 (segment (start 114.5 76.7) (end 120 76.7) (width 0.4) (layer "F.Cu") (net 8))
 (segment (start 126.6 76.7) (end 126.65 76.7) (width 0.4) (layer "F.Cu") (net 8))
 (segment (start 120 76.7) (end 126.6 76.7) (width 0.5) (layer "F.Cu") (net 8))
 (segment (start 128.35 75) (end 128.75 75) (width 0.4) (layer "F.Cu") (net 8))
 (segment (start 132.4 75) (end 134.1 76.7) (width 0.4) (layer "F.Cu") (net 7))
 (segment (start 134.1 76.7) (end 137 76.7) (width 0.4) (layer "F.Cu") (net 7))
 (segment (start 131.25 75) (end 132.4 75) (width 0.4) (layer "F.Cu") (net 7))
 (segment (start 120 72.2) (end 137 72.2) (width 0.4) (layer "F.Cu") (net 3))
 (segment (start 80 72.2) (end 100 72.2) (width 0.4) (layer "F.Cu") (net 3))
 (segment (start 60 72.2) (end 80 72.2) (width 0.4) (layer "F.Cu") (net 3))
 (segment (start 60 72.2) (end 43 72.2) (width 0.4) (layer "F.Cu") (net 3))
 (segment (start 100 72.2) (end 120 72.2) (width 0.4) (layer "F.Cu") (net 3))
 (segment (start 80 77.8) (end 100 77.8) (width 0.4) (layer "F.Cu") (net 5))
 (segment (start 100 77.8) (end 120 77.8) (width 0.4) (layer "F.Cu") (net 5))
 (segment (start 120.1 77.9) (end 136.9 77.9) (width 0.4) (layer "F.Cu") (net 5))
 (segment (start 43 77.8) (end 60 77.8) (width 0.4) (layer "F.Cu") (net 5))
 (segment (start 120 77.8) (end 120.1 77.9) (width 0.4) (layer "F.Cu") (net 5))
 (segment (start 136.9 77.9) (end 137 77.8) (width 0.4) (layer "F.Cu") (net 5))
 (segment (start 60 77.8) (end 80 77.8) (width 0.4) (layer "F.Cu") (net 5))
 (segment (start 47 75.175) (end 48.575 75.175) (width 0.4) (layer "F.Cu") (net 11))
 (segment (start 48.575 75.175) (end 48.75 75) (width 0.3) (layer "F.Cu") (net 11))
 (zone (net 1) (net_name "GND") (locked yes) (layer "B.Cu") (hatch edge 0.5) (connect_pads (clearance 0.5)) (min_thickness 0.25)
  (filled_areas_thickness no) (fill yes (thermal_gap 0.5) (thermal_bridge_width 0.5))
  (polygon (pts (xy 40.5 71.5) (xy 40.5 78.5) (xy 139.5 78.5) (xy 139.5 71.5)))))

